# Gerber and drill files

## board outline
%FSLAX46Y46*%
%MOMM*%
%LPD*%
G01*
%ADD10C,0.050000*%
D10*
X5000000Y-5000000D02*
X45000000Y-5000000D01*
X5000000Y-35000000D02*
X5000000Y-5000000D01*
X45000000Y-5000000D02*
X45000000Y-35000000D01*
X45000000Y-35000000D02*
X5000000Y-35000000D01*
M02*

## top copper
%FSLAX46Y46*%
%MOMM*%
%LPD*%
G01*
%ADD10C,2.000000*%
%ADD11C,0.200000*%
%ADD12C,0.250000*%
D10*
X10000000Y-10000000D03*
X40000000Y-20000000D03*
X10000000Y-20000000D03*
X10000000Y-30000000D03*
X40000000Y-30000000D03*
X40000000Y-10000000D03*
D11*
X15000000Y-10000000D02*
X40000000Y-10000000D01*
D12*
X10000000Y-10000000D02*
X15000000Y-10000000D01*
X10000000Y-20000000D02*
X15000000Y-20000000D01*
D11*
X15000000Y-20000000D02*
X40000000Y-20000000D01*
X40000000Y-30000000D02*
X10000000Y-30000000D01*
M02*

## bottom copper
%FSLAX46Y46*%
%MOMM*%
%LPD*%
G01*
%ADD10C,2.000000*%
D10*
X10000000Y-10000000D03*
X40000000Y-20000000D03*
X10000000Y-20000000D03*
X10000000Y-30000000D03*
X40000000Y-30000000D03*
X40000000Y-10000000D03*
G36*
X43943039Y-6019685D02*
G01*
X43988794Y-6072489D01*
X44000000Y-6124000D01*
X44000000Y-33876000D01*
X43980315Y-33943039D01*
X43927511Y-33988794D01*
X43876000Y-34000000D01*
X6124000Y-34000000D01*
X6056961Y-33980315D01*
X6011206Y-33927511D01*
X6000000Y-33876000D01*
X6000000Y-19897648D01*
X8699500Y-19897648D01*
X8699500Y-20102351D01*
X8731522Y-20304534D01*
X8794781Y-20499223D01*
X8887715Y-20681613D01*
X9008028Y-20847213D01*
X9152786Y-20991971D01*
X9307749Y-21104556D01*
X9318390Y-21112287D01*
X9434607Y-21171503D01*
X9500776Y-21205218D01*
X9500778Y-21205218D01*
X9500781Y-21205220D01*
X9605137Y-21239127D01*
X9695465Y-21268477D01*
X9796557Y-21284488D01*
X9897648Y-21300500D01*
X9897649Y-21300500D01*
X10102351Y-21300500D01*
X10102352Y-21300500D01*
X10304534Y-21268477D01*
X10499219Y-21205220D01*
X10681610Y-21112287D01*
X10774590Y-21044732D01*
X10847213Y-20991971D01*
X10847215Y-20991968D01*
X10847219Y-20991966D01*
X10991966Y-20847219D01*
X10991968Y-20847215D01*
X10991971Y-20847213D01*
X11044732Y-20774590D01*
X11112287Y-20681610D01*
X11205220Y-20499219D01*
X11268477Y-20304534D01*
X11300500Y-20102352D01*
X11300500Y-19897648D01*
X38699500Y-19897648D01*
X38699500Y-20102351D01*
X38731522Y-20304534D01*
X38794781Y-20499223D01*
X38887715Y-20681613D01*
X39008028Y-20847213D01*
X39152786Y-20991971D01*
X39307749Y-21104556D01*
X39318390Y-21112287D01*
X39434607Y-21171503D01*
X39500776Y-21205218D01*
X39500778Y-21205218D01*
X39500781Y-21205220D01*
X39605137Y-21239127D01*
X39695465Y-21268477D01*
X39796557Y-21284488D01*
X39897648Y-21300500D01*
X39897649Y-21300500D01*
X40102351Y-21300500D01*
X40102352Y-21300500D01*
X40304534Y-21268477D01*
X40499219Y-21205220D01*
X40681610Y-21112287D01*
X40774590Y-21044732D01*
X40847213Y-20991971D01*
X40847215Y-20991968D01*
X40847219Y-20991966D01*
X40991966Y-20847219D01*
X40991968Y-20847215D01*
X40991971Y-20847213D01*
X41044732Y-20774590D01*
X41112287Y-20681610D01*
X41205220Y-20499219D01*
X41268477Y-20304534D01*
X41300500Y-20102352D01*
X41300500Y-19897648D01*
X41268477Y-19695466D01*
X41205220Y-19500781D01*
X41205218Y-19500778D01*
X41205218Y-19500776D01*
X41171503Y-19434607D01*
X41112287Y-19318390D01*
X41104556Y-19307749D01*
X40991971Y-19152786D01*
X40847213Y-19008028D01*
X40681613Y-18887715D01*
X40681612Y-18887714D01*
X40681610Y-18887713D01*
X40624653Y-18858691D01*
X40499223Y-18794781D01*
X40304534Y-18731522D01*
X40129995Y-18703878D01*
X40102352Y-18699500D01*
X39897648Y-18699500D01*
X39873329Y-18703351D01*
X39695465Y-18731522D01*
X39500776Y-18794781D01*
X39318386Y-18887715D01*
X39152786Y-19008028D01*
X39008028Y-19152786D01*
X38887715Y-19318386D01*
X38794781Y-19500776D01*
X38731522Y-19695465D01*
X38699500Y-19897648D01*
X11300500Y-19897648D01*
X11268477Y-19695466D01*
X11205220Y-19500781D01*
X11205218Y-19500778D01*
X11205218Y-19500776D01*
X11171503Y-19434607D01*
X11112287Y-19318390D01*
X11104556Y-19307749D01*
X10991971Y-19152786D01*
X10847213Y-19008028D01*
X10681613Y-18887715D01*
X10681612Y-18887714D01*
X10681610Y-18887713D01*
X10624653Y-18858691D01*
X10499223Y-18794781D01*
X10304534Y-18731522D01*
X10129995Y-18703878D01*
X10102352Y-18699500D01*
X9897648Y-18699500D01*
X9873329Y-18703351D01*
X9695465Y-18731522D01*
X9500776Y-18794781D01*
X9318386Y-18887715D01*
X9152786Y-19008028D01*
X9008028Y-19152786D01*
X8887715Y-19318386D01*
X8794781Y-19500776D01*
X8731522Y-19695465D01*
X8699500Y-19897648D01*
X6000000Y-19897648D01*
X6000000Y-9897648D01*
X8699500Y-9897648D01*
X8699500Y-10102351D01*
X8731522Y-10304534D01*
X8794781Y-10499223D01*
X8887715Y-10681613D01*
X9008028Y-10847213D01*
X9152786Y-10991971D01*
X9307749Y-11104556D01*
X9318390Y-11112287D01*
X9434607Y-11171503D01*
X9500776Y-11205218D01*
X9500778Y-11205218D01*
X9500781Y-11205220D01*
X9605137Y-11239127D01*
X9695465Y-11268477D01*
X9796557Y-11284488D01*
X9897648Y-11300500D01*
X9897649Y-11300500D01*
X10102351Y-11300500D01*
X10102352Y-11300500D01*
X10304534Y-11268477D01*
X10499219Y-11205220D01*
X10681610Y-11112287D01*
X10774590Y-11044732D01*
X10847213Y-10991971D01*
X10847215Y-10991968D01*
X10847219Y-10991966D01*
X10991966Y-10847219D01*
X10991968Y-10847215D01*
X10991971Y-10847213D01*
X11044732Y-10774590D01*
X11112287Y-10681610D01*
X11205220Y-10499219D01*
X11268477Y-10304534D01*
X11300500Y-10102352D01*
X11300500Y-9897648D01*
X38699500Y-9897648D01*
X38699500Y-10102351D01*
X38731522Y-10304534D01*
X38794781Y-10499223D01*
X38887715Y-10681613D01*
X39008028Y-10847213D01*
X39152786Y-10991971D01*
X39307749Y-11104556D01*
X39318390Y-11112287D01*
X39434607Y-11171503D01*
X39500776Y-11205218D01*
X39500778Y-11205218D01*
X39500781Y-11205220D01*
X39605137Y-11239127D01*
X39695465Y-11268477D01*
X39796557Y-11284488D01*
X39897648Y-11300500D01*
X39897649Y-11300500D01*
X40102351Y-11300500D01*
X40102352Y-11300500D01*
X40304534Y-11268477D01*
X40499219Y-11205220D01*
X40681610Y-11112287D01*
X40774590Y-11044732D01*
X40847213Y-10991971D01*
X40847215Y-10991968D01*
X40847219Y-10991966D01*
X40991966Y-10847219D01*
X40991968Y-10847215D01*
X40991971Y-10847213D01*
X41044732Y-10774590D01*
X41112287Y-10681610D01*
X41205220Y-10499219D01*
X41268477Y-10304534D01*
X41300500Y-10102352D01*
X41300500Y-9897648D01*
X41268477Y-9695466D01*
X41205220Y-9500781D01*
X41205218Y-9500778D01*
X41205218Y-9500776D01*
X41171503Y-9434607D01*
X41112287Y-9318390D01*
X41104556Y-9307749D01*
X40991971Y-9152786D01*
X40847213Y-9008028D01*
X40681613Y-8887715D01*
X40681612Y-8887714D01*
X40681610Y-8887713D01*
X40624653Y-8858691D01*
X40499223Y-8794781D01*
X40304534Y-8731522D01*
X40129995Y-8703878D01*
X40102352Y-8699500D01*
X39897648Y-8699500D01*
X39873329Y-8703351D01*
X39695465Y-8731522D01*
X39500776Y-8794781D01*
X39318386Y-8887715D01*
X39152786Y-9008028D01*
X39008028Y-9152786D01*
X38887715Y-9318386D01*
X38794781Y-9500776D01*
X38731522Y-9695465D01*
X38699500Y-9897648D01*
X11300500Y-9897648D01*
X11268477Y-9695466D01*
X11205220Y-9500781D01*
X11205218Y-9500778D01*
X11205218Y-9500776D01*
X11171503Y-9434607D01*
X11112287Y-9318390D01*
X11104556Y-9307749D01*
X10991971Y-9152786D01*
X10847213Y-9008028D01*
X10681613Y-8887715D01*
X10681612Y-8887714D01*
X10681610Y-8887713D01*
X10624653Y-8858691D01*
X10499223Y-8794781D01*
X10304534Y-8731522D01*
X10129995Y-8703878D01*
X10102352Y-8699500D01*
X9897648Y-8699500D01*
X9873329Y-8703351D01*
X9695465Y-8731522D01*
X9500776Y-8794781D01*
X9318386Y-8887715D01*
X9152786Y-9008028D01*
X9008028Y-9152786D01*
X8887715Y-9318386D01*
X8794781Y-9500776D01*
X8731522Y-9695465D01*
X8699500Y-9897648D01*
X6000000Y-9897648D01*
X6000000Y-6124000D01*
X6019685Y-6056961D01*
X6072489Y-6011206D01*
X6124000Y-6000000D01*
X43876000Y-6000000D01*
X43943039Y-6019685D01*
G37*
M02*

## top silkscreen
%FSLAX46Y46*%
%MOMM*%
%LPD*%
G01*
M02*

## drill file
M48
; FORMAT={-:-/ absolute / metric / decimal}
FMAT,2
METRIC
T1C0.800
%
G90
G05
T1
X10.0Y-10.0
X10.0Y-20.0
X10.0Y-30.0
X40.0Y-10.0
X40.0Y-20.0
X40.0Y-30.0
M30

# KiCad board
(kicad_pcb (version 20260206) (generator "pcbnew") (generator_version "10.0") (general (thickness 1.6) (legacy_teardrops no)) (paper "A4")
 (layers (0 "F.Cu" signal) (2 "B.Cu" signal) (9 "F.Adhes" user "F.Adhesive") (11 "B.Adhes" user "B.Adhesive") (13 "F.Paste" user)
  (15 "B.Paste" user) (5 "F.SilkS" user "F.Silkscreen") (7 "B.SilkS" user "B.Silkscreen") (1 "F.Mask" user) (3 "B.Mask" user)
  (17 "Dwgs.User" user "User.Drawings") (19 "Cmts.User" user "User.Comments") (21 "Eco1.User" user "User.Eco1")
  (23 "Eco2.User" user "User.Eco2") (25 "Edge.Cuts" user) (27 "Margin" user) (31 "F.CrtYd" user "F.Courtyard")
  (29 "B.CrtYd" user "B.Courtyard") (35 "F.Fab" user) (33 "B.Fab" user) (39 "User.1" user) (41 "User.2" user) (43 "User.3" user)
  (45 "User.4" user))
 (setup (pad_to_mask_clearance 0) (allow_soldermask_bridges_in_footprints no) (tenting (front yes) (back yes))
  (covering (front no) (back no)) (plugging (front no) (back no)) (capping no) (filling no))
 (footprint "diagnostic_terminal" (layer "F.Cu") (at 10 10)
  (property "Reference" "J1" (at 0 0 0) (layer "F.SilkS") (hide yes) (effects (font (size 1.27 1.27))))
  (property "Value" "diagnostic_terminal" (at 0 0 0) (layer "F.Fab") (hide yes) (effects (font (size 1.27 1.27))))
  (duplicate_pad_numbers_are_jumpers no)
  (pad "1" thru_hole circle (at 0 0) (size 2 2) (drill 0.8) (layers "*.Cu") (remove_unused_layers no) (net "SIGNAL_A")))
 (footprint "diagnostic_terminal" (layer "F.Cu") (at 40 20)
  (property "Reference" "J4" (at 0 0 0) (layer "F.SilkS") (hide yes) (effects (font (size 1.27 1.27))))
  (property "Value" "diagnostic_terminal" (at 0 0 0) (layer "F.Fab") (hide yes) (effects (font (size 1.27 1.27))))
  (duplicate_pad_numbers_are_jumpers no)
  (pad "1" thru_hole circle (at 0 0) (size 2 2) (drill 0.8) (layers "*.Cu") (remove_unused_layers no) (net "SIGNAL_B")))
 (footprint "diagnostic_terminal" (layer "F.Cu") (at 10 20)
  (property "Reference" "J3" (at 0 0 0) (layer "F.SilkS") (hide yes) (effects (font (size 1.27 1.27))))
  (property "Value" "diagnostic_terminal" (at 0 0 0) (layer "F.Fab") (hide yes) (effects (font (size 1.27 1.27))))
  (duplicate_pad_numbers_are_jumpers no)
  (pad "1" thru_hole circle (at 0 0) (size 2 2) (drill 0.8) (layers "*.Cu") (remove_unused_layers no) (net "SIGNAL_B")))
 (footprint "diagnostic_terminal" (layer "F.Cu") (at 10 30)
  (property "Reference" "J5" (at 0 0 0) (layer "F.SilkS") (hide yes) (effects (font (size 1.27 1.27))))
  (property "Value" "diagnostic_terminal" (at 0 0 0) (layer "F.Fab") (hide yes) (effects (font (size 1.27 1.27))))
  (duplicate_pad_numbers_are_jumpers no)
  (pad "1" thru_hole circle (at 0 0) (size 2 2) (drill 0.8) (layers "*.Cu") (remove_unused_layers no) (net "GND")))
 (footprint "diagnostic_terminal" (layer "F.Cu") (at 40 30)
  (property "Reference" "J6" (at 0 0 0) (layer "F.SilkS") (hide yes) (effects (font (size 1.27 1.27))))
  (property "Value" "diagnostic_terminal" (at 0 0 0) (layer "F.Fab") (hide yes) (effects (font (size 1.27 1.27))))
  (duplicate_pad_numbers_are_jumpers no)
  (pad "1" thru_hole circle (at 0 0) (size 2 2) (drill 0.8) (layers "*.Cu") (remove_unused_layers no) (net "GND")))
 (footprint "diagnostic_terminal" (layer "F.Cu") (at 40 10)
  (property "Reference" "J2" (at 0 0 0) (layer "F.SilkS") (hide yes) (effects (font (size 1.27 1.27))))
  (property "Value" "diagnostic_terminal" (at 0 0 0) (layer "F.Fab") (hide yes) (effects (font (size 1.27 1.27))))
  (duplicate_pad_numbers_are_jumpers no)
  (pad "1" thru_hole circle (at 0 0) (size 2 2) (drill 0.8) (layers "*.Cu") (remove_unused_layers no) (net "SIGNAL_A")))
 (gr_line (start 5 5) (end 45 5) (stroke (width 0.05) (type default)) (layer "Edge.Cuts"))
 (gr_line (start 5 35) (end 5 5) (stroke (width 0.05) (type default)) (layer "Edge.Cuts"))
 (gr_line (start 45 5) (end 45 35) (stroke (width 0.05) (type default)) (layer "Edge.Cuts"))
 (gr_line (start 45 35) (end 5 35) (stroke (width 0.05) (type default)) (layer "Edge.Cuts"))
 (segment (start 15 10) (end 40 10) (width 0.2) (layer "F.Cu") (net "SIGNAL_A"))
 (segment (start 10 10) (end 15 10) (width 0.25) (locked yes) (layer "F.Cu") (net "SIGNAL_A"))
 (segment (start 10 20) (end 15 20) (width 0.25) (locked yes) (layer "F.Cu") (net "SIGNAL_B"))
 (segment (start 15 20) (end 40 20) (width 0.2) (layer "F.Cu") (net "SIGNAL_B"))
 (segment (start 40 30) (end 10 30) (width 0.2) (layer "F.Cu") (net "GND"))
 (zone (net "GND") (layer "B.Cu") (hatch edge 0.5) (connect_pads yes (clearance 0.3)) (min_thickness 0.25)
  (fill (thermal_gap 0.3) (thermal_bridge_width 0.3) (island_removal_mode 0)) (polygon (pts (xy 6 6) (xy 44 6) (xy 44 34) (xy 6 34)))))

